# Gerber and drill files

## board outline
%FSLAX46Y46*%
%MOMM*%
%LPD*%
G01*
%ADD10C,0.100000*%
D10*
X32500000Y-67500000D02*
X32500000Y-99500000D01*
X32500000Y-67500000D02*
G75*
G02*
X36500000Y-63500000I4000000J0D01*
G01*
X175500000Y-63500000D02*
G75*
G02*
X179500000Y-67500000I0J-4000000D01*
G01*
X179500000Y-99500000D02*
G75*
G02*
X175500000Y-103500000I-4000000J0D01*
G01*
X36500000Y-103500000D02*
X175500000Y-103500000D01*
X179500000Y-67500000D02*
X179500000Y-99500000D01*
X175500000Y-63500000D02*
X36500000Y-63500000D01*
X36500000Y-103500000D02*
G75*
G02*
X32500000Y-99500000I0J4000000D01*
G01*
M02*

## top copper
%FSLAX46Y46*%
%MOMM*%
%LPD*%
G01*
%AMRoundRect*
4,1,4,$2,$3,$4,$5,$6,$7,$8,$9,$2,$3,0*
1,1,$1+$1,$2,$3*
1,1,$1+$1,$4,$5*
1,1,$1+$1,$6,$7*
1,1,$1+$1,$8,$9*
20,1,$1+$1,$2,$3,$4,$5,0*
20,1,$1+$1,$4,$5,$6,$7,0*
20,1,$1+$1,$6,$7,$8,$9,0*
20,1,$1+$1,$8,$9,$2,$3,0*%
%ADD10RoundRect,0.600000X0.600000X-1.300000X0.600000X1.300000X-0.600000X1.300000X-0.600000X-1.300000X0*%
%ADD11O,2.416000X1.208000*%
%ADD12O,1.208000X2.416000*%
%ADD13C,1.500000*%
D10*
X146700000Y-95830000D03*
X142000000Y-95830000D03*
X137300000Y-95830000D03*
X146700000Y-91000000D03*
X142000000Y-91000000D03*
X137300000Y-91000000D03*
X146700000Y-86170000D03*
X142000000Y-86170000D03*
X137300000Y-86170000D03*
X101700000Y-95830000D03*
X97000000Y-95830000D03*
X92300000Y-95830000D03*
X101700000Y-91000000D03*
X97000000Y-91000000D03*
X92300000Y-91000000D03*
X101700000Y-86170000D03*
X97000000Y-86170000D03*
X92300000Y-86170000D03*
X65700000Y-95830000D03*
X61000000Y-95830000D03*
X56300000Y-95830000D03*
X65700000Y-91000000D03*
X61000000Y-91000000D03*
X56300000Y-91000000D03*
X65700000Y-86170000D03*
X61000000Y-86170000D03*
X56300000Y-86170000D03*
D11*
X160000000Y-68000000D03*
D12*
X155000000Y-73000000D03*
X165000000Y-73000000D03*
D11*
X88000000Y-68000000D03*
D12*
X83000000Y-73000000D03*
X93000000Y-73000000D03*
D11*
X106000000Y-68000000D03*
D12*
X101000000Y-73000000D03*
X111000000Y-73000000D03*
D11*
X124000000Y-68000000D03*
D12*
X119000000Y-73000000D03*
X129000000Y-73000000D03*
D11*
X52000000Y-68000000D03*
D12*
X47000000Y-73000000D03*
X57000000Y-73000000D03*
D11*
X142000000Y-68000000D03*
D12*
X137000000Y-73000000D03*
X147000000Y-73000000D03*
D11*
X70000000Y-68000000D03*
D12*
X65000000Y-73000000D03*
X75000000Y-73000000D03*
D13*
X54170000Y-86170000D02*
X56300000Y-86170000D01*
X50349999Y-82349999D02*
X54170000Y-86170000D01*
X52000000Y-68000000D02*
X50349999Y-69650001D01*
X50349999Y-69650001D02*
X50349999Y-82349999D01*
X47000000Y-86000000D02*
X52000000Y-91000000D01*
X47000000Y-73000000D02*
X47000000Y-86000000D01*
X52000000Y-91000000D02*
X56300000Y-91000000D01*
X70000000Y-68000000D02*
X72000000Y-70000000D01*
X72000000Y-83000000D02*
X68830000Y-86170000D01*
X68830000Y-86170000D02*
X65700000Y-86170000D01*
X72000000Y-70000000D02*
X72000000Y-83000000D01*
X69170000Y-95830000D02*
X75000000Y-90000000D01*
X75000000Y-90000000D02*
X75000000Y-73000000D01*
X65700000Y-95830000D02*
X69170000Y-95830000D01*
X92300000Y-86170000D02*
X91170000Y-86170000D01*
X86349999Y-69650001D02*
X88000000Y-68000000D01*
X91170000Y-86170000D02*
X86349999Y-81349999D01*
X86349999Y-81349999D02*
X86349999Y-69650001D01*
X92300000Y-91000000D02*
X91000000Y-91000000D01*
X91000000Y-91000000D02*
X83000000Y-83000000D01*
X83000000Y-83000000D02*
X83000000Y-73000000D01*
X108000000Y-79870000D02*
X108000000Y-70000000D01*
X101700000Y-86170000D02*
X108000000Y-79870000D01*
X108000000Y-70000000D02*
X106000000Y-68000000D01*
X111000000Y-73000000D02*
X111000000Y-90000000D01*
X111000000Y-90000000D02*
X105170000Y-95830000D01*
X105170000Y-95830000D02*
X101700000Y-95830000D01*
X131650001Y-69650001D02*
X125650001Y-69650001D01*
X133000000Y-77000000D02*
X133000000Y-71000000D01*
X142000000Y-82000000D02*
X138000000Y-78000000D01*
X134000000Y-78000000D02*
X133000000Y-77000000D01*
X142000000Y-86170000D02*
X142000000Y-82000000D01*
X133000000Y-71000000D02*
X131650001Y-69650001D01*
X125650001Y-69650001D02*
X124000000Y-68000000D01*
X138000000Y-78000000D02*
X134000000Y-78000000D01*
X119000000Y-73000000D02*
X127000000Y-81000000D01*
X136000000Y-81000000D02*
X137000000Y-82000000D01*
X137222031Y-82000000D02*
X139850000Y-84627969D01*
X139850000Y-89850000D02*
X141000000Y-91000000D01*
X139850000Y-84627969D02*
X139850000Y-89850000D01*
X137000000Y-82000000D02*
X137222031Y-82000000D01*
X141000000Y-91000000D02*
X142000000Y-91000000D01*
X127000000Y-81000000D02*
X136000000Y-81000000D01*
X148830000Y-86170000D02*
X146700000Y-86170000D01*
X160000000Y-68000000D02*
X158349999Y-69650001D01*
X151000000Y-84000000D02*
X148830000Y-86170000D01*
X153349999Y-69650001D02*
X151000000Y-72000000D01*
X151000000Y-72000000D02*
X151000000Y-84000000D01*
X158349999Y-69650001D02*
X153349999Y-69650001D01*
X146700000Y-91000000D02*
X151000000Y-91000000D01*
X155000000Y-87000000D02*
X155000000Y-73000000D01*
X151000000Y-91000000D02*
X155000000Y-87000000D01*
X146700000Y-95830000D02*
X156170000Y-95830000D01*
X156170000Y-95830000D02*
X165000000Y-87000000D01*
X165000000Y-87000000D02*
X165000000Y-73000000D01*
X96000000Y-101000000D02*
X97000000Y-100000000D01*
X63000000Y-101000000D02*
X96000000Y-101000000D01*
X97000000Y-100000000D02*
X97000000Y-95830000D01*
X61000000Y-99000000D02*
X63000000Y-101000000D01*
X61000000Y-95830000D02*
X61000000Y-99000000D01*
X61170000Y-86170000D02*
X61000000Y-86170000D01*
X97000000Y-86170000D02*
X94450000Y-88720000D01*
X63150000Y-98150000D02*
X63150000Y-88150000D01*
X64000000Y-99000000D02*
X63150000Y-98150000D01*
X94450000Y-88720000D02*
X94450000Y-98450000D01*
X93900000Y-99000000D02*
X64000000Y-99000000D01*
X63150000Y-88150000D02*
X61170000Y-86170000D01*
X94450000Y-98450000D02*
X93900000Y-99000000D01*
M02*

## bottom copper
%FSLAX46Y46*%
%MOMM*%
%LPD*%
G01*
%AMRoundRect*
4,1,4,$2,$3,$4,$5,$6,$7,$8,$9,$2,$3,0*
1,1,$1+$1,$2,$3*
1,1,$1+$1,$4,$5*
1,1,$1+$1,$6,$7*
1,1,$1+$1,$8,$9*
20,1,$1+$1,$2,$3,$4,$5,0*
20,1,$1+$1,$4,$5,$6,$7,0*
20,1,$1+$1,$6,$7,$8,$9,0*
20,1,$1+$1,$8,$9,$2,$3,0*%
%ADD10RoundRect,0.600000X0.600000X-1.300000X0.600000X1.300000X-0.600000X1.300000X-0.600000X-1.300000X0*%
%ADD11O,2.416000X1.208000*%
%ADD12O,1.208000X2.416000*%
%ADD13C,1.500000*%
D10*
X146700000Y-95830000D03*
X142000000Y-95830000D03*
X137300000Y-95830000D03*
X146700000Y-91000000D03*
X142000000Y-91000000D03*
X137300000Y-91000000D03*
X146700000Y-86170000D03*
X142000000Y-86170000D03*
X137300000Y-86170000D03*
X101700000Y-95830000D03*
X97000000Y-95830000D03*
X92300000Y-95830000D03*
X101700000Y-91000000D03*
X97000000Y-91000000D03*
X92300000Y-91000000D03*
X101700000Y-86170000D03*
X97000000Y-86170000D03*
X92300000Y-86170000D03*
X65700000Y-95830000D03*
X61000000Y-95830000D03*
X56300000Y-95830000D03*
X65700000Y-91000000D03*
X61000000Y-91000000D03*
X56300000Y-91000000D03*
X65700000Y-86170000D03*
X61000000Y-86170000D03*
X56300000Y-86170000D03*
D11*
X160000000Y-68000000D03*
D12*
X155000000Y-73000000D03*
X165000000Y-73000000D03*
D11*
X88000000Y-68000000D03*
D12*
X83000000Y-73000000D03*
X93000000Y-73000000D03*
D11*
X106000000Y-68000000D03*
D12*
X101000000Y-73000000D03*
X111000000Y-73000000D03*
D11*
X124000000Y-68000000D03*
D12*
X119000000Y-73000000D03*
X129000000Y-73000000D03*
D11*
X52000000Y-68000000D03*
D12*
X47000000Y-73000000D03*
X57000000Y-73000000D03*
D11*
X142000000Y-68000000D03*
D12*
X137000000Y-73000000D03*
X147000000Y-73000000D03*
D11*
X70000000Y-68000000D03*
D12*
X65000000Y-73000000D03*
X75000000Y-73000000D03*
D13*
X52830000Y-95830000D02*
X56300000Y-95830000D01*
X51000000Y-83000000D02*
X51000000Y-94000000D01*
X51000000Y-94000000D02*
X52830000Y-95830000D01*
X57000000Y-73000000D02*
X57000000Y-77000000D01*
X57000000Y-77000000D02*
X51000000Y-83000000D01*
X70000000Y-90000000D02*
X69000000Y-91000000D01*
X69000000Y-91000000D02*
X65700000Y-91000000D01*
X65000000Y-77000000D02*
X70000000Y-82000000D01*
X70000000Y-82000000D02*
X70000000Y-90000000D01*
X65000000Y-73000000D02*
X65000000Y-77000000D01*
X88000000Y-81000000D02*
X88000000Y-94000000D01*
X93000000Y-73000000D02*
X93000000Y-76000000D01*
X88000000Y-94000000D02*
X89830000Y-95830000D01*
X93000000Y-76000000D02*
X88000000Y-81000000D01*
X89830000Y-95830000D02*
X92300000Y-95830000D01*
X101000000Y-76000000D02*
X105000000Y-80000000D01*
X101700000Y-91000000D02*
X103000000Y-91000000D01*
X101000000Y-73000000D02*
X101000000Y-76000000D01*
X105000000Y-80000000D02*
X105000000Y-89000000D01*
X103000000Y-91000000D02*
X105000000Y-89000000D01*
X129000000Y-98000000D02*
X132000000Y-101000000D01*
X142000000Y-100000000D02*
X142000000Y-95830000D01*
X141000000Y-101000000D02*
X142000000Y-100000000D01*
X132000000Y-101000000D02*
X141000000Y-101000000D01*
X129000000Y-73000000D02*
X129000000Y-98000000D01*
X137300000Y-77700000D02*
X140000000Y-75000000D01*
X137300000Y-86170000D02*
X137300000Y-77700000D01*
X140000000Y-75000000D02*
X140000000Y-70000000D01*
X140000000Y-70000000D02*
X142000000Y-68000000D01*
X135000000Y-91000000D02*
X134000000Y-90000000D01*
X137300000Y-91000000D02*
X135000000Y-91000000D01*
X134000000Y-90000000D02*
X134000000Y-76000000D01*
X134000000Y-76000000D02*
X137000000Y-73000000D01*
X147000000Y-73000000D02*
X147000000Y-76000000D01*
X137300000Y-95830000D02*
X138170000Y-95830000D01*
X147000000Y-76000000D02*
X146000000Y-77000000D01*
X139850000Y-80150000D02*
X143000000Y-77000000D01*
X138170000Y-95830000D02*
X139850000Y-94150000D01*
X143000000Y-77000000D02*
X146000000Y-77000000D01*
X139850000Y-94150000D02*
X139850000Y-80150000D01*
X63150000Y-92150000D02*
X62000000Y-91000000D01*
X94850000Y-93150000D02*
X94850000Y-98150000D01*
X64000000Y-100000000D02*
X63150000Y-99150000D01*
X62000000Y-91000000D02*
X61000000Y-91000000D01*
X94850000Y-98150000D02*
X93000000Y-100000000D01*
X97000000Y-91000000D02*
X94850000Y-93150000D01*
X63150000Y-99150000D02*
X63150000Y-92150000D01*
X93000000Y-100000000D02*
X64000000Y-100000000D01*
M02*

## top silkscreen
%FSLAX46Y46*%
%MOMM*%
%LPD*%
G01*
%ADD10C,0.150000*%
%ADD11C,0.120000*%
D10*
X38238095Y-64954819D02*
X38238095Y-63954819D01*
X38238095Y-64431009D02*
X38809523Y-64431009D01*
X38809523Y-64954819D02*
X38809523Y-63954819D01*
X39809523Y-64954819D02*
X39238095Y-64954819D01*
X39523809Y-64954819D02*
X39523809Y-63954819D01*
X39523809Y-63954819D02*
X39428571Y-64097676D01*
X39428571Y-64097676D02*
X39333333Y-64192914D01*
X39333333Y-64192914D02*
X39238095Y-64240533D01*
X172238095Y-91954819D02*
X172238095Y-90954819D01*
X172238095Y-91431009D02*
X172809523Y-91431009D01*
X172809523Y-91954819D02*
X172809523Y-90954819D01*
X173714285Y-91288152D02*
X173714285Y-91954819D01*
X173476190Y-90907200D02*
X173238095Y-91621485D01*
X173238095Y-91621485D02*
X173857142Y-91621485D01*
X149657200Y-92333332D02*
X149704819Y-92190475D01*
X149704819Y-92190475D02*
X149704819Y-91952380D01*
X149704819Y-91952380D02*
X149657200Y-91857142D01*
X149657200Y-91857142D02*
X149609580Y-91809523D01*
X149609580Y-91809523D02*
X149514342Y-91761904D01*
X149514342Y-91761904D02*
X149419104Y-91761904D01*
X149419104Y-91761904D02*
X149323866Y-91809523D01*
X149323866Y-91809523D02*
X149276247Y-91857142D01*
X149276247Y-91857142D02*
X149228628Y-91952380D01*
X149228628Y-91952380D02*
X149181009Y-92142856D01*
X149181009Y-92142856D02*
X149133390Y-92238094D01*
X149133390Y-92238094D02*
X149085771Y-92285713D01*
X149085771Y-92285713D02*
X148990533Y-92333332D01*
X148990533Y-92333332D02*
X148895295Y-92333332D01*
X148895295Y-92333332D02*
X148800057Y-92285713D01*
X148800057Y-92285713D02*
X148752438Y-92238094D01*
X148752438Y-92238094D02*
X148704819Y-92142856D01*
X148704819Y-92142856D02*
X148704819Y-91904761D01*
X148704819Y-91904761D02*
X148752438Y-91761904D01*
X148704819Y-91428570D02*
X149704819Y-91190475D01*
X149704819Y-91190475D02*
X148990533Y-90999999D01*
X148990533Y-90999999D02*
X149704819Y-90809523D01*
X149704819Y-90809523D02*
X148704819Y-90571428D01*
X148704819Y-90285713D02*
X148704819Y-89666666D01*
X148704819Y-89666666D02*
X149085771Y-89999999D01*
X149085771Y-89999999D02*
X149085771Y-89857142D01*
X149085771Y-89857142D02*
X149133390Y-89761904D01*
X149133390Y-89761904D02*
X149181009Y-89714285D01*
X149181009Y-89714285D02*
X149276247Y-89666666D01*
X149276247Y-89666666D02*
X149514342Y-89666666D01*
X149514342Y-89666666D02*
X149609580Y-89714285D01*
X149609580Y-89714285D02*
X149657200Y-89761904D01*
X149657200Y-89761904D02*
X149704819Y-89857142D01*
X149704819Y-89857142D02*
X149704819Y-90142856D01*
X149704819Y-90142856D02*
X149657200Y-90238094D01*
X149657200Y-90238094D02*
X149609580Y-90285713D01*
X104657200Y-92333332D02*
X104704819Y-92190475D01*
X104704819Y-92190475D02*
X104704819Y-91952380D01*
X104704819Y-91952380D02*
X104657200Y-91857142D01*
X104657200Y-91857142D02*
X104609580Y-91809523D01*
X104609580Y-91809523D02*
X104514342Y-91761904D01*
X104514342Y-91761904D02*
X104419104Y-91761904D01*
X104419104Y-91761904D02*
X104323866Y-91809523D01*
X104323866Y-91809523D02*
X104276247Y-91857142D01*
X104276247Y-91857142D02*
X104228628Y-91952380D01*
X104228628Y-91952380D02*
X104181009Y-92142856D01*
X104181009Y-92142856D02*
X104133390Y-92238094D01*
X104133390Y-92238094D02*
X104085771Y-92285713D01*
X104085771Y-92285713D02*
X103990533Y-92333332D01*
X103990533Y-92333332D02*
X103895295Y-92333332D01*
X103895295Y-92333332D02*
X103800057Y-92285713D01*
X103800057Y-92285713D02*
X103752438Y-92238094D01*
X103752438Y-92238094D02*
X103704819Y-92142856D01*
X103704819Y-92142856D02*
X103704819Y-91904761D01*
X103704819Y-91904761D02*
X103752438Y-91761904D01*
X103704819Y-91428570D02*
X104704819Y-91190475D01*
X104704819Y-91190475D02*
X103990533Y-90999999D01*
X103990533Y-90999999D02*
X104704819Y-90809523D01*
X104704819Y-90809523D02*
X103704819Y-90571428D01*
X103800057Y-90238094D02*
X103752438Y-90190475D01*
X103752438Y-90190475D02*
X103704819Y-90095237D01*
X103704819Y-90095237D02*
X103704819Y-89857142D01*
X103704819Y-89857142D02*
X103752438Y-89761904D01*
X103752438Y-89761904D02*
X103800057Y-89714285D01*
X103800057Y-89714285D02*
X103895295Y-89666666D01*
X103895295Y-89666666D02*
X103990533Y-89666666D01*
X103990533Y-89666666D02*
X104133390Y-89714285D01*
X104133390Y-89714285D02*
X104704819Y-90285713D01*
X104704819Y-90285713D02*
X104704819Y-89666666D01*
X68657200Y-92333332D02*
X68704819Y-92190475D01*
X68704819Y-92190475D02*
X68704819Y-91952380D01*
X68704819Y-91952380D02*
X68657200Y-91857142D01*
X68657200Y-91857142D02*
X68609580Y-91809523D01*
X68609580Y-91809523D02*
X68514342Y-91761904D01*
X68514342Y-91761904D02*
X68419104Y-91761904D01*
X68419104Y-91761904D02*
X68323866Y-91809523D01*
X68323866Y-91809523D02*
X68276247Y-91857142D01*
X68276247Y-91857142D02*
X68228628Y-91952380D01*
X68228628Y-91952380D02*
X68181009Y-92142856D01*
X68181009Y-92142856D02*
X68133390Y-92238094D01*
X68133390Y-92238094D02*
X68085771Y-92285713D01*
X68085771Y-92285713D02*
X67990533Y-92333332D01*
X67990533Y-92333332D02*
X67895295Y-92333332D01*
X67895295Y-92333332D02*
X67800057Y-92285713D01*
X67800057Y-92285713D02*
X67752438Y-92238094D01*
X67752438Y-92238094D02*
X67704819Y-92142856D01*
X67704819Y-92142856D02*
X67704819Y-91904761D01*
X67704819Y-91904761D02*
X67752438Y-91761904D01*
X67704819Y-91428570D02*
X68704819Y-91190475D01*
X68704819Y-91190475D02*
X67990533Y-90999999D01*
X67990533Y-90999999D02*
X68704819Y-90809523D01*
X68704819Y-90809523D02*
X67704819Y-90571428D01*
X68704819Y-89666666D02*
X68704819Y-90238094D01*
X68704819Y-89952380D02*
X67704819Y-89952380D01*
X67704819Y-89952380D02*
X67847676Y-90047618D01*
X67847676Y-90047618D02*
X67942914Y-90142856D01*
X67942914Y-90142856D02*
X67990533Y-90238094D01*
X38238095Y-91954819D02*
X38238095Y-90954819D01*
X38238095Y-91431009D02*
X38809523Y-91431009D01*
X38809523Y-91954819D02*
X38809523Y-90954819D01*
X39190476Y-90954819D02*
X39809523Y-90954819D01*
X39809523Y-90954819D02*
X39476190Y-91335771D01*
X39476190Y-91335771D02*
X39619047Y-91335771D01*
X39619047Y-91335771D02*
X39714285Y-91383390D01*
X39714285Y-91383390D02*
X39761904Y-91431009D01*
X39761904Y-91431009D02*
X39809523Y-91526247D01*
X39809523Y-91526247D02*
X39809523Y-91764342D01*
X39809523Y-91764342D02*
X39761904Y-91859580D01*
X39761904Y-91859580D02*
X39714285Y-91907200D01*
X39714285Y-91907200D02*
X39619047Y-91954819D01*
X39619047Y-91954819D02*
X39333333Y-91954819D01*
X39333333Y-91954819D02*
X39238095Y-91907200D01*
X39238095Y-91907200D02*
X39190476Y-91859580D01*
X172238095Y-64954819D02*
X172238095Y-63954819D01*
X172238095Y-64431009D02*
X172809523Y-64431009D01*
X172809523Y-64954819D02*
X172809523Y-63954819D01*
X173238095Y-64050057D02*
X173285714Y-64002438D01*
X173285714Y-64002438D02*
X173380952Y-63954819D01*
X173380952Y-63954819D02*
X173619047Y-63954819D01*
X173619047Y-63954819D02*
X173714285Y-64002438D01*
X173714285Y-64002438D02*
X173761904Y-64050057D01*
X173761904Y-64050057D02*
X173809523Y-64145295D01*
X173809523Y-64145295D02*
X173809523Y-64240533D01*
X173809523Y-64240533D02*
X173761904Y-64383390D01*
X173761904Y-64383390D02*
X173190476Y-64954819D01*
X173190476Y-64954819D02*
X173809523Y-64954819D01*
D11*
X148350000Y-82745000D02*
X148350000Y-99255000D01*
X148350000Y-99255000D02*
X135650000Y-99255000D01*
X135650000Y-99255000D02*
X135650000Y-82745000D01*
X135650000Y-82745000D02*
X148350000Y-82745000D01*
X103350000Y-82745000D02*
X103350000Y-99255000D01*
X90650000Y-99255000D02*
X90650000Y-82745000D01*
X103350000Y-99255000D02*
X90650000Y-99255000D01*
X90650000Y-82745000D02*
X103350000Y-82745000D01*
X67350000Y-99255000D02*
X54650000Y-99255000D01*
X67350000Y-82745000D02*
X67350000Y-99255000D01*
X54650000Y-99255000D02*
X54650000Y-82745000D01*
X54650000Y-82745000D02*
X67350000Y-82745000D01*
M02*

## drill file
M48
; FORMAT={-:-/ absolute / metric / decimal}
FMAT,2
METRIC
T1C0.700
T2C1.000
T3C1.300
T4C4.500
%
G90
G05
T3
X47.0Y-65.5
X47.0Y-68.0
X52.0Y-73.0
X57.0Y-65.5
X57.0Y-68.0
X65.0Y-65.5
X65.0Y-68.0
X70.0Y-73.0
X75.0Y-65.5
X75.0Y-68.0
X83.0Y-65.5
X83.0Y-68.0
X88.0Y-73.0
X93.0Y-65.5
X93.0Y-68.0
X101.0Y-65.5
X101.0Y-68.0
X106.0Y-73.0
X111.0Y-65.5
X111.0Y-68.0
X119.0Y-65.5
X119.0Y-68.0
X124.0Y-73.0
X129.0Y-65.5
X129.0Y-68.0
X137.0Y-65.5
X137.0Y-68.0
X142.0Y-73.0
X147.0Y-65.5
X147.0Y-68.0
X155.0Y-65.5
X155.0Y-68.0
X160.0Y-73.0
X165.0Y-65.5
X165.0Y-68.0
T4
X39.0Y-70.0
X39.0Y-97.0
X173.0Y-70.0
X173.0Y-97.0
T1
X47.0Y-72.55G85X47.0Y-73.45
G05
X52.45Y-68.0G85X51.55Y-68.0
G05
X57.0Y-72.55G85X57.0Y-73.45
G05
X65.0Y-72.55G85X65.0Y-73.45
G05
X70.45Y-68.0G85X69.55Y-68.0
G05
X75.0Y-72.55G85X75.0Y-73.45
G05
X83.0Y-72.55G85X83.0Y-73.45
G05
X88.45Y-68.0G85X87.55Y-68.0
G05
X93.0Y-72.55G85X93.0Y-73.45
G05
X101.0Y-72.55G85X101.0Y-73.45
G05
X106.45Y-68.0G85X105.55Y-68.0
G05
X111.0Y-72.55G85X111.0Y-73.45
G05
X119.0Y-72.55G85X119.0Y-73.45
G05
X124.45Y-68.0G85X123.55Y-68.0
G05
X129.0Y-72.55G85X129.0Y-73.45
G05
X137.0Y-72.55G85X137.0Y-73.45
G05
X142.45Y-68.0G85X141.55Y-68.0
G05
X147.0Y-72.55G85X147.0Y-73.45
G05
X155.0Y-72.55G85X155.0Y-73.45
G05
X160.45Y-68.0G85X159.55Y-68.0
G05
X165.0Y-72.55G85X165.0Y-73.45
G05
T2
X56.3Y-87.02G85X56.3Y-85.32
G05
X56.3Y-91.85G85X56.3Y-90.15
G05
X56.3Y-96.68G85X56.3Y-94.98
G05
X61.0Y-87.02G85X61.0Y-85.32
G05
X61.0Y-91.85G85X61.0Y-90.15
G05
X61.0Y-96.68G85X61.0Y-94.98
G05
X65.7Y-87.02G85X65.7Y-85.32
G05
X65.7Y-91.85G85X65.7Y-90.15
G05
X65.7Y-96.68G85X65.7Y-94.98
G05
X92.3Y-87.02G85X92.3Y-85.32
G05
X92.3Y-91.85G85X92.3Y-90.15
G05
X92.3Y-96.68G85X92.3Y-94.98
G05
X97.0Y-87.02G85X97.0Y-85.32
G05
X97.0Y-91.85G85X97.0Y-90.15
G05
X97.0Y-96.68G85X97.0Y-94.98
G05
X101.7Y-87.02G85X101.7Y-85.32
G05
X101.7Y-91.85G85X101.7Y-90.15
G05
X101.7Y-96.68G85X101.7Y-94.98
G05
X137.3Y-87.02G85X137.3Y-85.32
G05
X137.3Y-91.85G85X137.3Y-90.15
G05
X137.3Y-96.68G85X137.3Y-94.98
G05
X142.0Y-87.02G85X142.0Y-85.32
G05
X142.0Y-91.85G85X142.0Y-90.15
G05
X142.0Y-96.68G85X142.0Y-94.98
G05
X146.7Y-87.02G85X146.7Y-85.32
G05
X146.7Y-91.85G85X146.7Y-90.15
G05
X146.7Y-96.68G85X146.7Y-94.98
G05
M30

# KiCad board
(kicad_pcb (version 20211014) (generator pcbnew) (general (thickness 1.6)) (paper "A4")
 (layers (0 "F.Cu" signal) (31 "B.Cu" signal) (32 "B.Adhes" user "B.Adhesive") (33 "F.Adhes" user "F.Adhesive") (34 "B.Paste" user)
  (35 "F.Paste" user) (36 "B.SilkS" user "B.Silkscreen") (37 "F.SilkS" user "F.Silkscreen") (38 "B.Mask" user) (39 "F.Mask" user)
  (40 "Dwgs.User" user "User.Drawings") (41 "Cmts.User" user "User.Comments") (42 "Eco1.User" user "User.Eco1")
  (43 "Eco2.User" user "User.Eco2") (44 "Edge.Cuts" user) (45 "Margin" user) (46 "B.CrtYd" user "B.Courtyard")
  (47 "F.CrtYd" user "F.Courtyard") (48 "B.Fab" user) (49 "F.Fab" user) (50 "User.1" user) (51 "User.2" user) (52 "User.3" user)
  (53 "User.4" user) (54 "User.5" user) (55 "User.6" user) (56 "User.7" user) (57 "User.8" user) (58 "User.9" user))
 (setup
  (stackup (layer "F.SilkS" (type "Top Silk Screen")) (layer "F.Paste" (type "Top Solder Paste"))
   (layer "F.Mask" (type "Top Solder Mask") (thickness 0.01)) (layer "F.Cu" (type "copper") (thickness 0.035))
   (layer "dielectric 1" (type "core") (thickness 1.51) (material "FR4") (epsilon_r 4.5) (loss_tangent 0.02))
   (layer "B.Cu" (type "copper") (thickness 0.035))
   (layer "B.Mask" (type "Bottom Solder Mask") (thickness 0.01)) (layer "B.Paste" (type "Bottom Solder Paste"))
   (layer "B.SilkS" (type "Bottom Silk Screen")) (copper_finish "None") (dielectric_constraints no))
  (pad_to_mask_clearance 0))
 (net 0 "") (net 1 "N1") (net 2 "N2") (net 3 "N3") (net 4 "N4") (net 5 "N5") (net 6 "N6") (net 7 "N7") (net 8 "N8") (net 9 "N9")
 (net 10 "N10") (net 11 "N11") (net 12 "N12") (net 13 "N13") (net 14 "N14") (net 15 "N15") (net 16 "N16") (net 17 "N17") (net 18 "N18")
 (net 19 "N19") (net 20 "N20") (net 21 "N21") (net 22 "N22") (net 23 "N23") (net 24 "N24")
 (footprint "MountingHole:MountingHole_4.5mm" (layer "F.Cu") (at 39 70)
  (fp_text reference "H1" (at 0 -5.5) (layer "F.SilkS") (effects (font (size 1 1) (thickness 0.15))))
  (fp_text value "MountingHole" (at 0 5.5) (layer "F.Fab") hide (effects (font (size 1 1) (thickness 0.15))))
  (pad "" np_thru_hole circle (at 0 0) (size 4.5 4.5) (drill 4.5) (layers *.Cu *.Mask)))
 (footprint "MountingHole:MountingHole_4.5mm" (layer "F.Cu") (at 173 97)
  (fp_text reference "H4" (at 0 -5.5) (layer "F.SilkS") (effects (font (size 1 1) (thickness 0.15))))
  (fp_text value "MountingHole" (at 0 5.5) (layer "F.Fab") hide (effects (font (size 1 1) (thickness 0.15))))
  (pad "" np_thru_hole circle (at 0 0) (size 4.5 4.5) (drill 4.5) (layers *.Cu *.Mask)))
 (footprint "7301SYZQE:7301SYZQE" (layer "F.Cu") (at 142 91 90)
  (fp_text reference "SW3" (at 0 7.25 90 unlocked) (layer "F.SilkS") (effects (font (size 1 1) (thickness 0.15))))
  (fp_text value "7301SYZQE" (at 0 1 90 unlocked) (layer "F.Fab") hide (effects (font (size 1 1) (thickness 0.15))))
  (fp_line (start 8.255 6.35) (end -8.255 6.35) (layer "F.SilkS") (width 0.12))
  (fp_line (start -8.255 6.35) (end -8.255 -6.35) (layer "F.SilkS") (width 0.12))
  (fp_line (start -8.255 -6.35) (end 8.255 -6.35) (layer "F.SilkS") (width 0.12))
  (fp_line (start 8.255 -6.35) (end 8.255 6.35) (layer "F.SilkS") (width 0.12))
  (pad "1" thru_hole roundrect (at -4.83 4.7 90) (size 3.8 2.4) (drill oval 2.7 1) (layers *.Cu *.Mask) (roundrect_rratio 0.25) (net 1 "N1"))
  (pad "2" thru_hole roundrect (at -4.83 0 90) (size 3.8 2.4) (drill oval 2.7 1) (layers *.Cu *.Mask) (roundrect_rratio 0.25) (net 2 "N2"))
  (pad "3" thru_hole roundrect (at -4.83 -4.7 90) (size 3.8 2.4) (drill oval 2.7 1) (layers *.Cu *.Mask) (roundrect_rratio 0.25)
   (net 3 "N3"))
  (pad "4" thru_hole roundrect (at 0 4.7 90) (size 3.8 2.4) (drill oval 2.7 1) (layers *.Cu *.Mask) (roundrect_rratio 0.25) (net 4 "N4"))
  (pad "5" thru_hole roundrect (at 0 0 90) (size 3.8 2.4) (drill oval 2.7 1) (layers *.Cu *.Mask) (roundrect_rratio 0.25) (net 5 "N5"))
  (pad "6" thru_hole roundrect (at 0 -4.7 90) (size 3.8 2.4) (drill oval 2.7 1) (layers *.Cu *.Mask) (roundrect_rratio 0.25) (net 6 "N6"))
  (pad "7" thru_hole roundrect (at 4.83 4.7 90) (size 3.8 2.4) (drill oval 2.7 1) (layers *.Cu *.Mask) (roundrect_rratio 0.25) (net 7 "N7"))
  (pad "8" thru_hole roundrect (at 4.83 0 90) (size 3.8 2.4) (drill oval 2.7 1) (layers *.Cu *.Mask) (roundrect_rratio 0.25) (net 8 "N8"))
  (pad "9" thru_hole roundrect (at 4.83 -4.7 90) (size 3.8 2.4) (drill oval 2.7 1) (layers *.Cu *.Mask) (roundrect_rratio 0.25) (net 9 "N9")))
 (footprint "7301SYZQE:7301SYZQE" (layer "F.Cu") (at 97 91 90)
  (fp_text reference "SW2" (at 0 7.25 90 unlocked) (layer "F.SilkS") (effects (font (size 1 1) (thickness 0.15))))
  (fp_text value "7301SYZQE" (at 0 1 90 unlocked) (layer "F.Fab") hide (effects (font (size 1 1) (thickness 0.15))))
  (fp_line (start 8.255 6.35) (end -8.255 6.35) (layer "F.SilkS") (width 0.12))
  (fp_line (start -8.255 -6.35) (end 8.255 -6.35) (layer "F.SilkS") (width 0.12))
  (fp_line (start -8.255 6.35) (end -8.255 -6.35) (layer "F.SilkS") (width 0.12))
  (fp_line (start 8.255 -6.35) (end 8.255 6.35) (layer "F.SilkS") (width 0.12))
  (pad "1" thru_hole roundrect (at -4.83 4.7 90) (size 3.8 2.4) (drill oval 2.7 1) (layers *.Cu *.Mask) (roundrect_rratio 0.25)
   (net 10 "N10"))
  (pad "2" thru_hole roundrect (at -4.83 0 90) (size 3.8 2.4) (drill oval 2.7 1) (layers *.Cu *.Mask) (roundrect_rratio 0.25) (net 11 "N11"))
  (pad "3" thru_hole roundrect (at -4.83 -4.7 90) (size 3.8 2.4) (drill oval 2.7 1) (layers *.Cu *.Mask) (roundrect_rratio 0.25)
   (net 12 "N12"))
  (pad "4" thru_hole roundrect (at 0 4.7 90) (size 3.8 2.4) (drill oval 2.7 1) (layers *.Cu *.Mask) (roundrect_rratio 0.25) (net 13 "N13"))
  (pad "5" thru_hole roundrect (at 0 0 90) (size 3.8 2.4) (drill oval 2.7 1) (layers *.Cu *.Mask) (roundrect_rratio 0.25) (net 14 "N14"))
  (pad "6" thru_hole roundrect (at 0 -4.7 90) (size 3.8 2.4) (drill oval 2.7 1) (layers *.Cu *.Mask) (roundrect_rratio 0.25) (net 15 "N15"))
  (pad "7" thru_hole roundrect (at 4.83 4.7 90) (size 3.8 2.4) (drill oval 2.7 1) (layers *.Cu *.Mask) (roundrect_rratio 0.25)
   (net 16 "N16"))
  (pad "8" thru_hole roundrect (at 4.83 0 90) (size 3.8 2.4) (drill oval 2.7 1) (layers *.Cu *.Mask) (roundrect_rratio 0.25) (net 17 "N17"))
  (pad "9" thru_hole roundrect (at 4.83 -4.7 90) (size 3.8 2.4) (drill oval 2.7 1) (layers *.Cu *.Mask) (roundrect_rratio 0.25)
   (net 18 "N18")))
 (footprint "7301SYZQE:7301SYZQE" (layer "F.Cu") (at 61 91 90)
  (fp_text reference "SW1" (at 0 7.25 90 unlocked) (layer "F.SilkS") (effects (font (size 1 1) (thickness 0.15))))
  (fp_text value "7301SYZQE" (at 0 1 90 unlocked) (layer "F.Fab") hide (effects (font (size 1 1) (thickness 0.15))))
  (fp_line (start -8.255 6.35) (end -8.255 -6.35) (layer "F.SilkS") (width 0.12))
  (fp_line (start 8.255 6.35) (end -8.255 6.35) (layer "F.SilkS") (width 0.12))
  (fp_line (start -8.255 -6.35) (end 8.255 -6.35) (layer "F.SilkS") (width 0.12))
  (fp_line (start 8.255 -6.35) (end 8.255 6.35) (layer "F.SilkS") (width 0.12))
  (pad "1" thru_hole roundrect (at -4.83 4.7 90) (size 3.8 2.4) (drill oval 2.7 1) (layers *.Cu *.Mask) (roundrect_rratio 0.25)
   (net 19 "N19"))
  (pad "2" thru_hole roundrect (at -4.83 0 90) (size 3.8 2.4) (drill oval 2.7 1) (layers *.Cu *.Mask) (roundrect_rratio 0.25) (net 11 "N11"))
  (pad "3" thru_hole roundrect (at -4.83 -4.7 90) (size 3.8 2.4) (drill oval 2.7 1) (layers *.Cu *.Mask) (roundrect_rratio 0.25)
   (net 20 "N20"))
  (pad "4" thru_hole roundrect (at 0 4.7 90) (size 3.8 2.4) (drill oval 2.7 1) (layers *.Cu *.Mask) (roundrect_rratio 0.25) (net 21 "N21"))
  (pad "5" thru_hole roundrect (at 0 0 90) (size 3.8 2.4) (drill oval 2.7 1) (layers *.Cu *.Mask) (roundrect_rratio 0.25) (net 14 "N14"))
  (pad "6" thru_hole roundrect (at 0 -4.7 90) (size 3.8 2.4) (drill oval 2.7 1) (layers *.Cu *.Mask) (roundrect_rratio 0.25) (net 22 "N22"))
  (pad "7" thru_hole roundrect (at 4.83 4.7 90) (size 3.8 2.4) (drill oval 2.7 1) (layers *.Cu *.Mask) (roundrect_rratio 0.25)
   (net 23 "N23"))
  (pad "8" thru_hole roundrect (at 4.83 0 90) (size 3.8 2.4) (drill oval 2.7 1) (layers *.Cu *.Mask) (roundrect_rratio 0.25) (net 17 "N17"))
  (pad "9" thru_hole roundrect (at 4.83 -4.7 90) (size 3.8 2.4) (drill oval 2.7 1) (layers *.Cu *.Mask) (roundrect_rratio 0.25)
   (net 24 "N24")))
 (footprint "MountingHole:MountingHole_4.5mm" (layer "F.Cu") (at 39 97)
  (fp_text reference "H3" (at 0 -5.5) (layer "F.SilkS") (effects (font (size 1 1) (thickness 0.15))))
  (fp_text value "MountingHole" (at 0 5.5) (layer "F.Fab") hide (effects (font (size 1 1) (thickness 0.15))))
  (pad "" np_thru_hole circle (at 0 0) (size 4.5 4.5) (drill 4.5) (layers *.Cu *.Mask)))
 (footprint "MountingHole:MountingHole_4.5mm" (layer "F.Cu") (at 173 70)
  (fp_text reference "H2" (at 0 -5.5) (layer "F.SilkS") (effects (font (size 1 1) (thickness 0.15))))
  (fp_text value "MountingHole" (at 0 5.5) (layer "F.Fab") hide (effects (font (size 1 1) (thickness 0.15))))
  (pad "" np_thru_hole circle (at 0 0) (size 4.5 4.5) (drill 4.5) (layers *.Cu *.Mask)))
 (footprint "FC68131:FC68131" (layer "B.Cu") (at 160 68 -90)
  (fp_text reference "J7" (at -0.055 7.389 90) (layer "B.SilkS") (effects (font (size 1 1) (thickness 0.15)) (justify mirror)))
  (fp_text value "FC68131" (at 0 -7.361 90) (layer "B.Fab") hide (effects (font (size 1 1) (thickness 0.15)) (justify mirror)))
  (pad "" np_thru_hole circle (at 0 5 270) (size 1.3 1.3) (drill 1.3) (layers *.Cu *.Mask))
  (pad "" np_thru_hole circle (at 5 0 270) (size 1.3 1.3) (drill 1.3) (layers *.Cu *.Mask))
  (pad "" np_thru_hole circle (at 0 -5 270) (size 1.3 1.3) (drill 1.3) (layers *.Cu *.Mask))
  (pad "" np_thru_hole circle (at -2.5 -5 270) (size 1.3 1.3) (drill 1.3) (layers *.Cu *.Mask))
  (pad "" np_thru_hole circle (at -2.5 5 270) (size 1.3 1.3) (drill 1.3) (layers *.Cu *.Mask))
  (pad "1" thru_hole oval (at 0 0 270) (size 1.208 2.416) (drill oval 0.7 1.6) (layers *.Cu *.Mask) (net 7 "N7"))
  (pad "2" thru_hole oval (at 5 5 270) (size 2.416 1.208) (drill oval 1.6 0.7) (layers *.Cu *.Mask) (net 4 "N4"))
  (pad "5" thru_hole oval (at 5 -5 270) (size 2.416 1.208) (drill oval 1.6 0.7) (layers *.Cu *.Mask) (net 1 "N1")))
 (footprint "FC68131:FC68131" (layer "B.Cu") (at 88 68 -90)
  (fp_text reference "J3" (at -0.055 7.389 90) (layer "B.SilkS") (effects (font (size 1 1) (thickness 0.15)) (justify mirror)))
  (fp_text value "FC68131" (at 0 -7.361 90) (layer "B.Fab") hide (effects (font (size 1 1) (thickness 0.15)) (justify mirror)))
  (pad "" np_thru_hole circle (at -2.5 -5 270) (size 1.3 1.3) (drill 1.3) (layers *.Cu *.Mask))
  (pad "" np_thru_hole circle (at 5 0 270) (size 1.3 1.3) (drill 1.3) (layers *.Cu *.Mask))
  (pad "" np_thru_hole circle (at -2.5 5 270) (size 1.3 1.3) (drill 1.3) (layers *.Cu *.Mask))
  (pad "" np_thru_hole circle (at 0 -5 270) (size 1.3 1.3) (drill 1.3) (layers *.Cu *.Mask))
  (pad "" np_thru_hole circle (at 0 5 270) (size 1.3 1.3) (drill 1.3) (layers *.Cu *.Mask))
  (pad "1" thru_hole oval (at 0 0 270) (size 1.208 2.416) (drill oval 0.7 1.6) (layers *.Cu *.Mask) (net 18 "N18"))
  (pad "2" thru_hole oval (at 5 5 270) (size 2.416 1.208) (drill oval 1.6 0.7) (layers *.Cu *.Mask) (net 15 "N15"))
  (pad "5" thru_hole oval (at 5 -5 270) (size 2.416 1.208) (drill oval 1.6 0.7) (layers *.Cu *.Mask) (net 12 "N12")))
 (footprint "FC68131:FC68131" (layer "B.Cu") (at 106 68 -90)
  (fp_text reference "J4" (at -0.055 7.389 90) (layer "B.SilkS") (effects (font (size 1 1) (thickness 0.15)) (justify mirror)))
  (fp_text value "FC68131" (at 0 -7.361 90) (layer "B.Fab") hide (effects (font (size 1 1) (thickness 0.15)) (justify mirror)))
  (pad "" np_thru_hole circle (at 0 -5 270) (size 1.3 1.3) (drill 1.3) (layers *.Cu *.Mask))
  (pad "" np_thru_hole circle (at -2.5 5 270) (size 1.3 1.3) (drill 1.3) (layers *.Cu *.Mask))
  (pad "" np_thru_hole circle (at 0 5 270) (size 1.3 1.3) (drill 1.3) (layers *.Cu *.Mask))
  (pad "" np_thru_hole circle (at 5 0 270) (size 1.3 1.3) (drill 1.3) (layers *.Cu *.Mask))
  (pad "" np_thru_hole circle (at -2.5 -5 270) (size 1.3 1.3) (drill 1.3) (layers *.Cu *.Mask))
  (pad "1" thru_hole oval (at 0 0 270) (size 1.208 2.416) (drill oval 0.7 1.6) (layers *.Cu *.Mask) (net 16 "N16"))
  (pad "2" thru_hole oval (at 5 5 270) (size 2.416 1.208) (drill oval 1.6 0.7) (layers *.Cu *.Mask) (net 13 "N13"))
  (pad "5" thru_hole oval (at 5 -5 270) (size 2.416 1.208) (drill oval 1.6 0.7) (layers *.Cu *.Mask) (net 10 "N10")))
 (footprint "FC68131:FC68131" (layer "B.Cu") (at 124 68 -90)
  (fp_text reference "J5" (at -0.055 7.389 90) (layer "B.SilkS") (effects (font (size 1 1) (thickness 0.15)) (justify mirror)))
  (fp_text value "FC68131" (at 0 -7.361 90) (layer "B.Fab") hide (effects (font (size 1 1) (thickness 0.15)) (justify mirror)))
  (pad "" np_thru_hole circle (at 5 0 270) (size 1.3 1.3) (drill 1.3) (layers *.Cu *.Mask))
  (pad "" np_thru_hole circle (at 0 -5 270) (size 1.3 1.3) (drill 1.3) (layers *.Cu *.Mask))
  (pad "" np_thru_hole circle (at 0 5 270) (size 1.3 1.3) (drill 1.3) (layers *.Cu *.Mask))
  (pad "" np_thru_hole circle (at -2.5 -5 270) (size 1.3 1.3) (drill 1.3) (layers *.Cu *.Mask))
  (pad "" np_thru_hole circle (at -2.5 5 270) (size 1.3 1.3) (drill 1.3) (layers *.Cu *.Mask))
  (pad "1" thru_hole oval (at 0 0 270) (size 1.208 2.416) (drill oval 0.7 1.6) (layers *.Cu *.Mask) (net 8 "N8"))
  (pad "2" thru_hole oval (at 5 5 270) (size 2.416 1.208) (drill oval 1.6 0.7) (layers *.Cu *.Mask) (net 5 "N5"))
  (pad "5" thru_hole oval (at 5 -5 270) (size 2.416 1.208) (drill oval 1.6 0.7) (layers *.Cu *.Mask) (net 2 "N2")))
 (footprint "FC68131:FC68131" (layer "B.Cu") (at 52 68 -90)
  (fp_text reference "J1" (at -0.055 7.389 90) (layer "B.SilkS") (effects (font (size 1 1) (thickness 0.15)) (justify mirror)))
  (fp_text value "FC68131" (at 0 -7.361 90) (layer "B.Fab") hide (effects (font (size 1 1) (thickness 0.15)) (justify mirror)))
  (pad "" np_thru_hole circle (at 0 5 270) (size 1.3 1.3) (drill 1.3) (layers *.Cu *.Mask))
  (pad "" np_thru_hole circle (at -2.5 -5 270) (size 1.3 1.3) (drill 1.3) (layers *.Cu *.Mask))
  (pad "" np_thru_hole circle (at -2.5 5 270) (size 1.3 1.3) (drill 1.3) (layers *.Cu *.Mask))
  (pad "" np_thru_hole circle (at 0 -5 270) (size 1.3 1.3) (drill 1.3) (layers *.Cu *.Mask))
  (pad "" np_thru_hole circle (at 5 0 270) (size 1.3 1.3) (drill 1.3) (layers *.Cu *.Mask))
  (pad "1" thru_hole oval (at 0 0 270) (size 1.208 2.416) (drill oval 0.7 1.6) (layers *.Cu *.Mask) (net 24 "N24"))
  (pad "2" thru_hole oval (at 5 5 270) (size 2.416 1.208) (drill oval 1.6 0.7) (layers *.Cu *.Mask) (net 22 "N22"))
  (pad "5" thru_hole oval (at 5 -5 270) (size 2.416 1.208) (drill oval 1.6 0.7) (layers *.Cu *.Mask) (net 20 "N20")))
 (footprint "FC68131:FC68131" (layer "B.Cu") (at 142 68 -90)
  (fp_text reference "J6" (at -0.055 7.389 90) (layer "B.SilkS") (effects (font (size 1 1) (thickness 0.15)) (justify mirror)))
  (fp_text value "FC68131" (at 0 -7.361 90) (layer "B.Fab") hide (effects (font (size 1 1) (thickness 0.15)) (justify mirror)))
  (pad "" np_thru_hole circle (at 0 5 270) (size 1.3 1.3) (drill 1.3) (layers *.Cu *.Mask))
  (pad "" np_thru_hole circle (at 0 -5 270) (size 1.3 1.3) (drill 1.3) (layers *.Cu *.Mask))
  (pad "" np_thru_hole circle (at -2.5 5 270) (size 1.3 1.3) (drill 1.3) (layers *.Cu *.Mask))
  (pad "" np_thru_hole circle (at -2.5 -5 270) (size 1.3 1.3) (drill 1.3) (layers *.Cu *.Mask))
  (pad "" np_thru_hole circle (at 5 0 270) (size 1.3 1.3) (drill 1.3) (layers *.Cu *.Mask))
  (pad "1" thru_hole oval (at 0 0 270) (size 1.208 2.416) (drill oval 0.7 1.6) (layers *.Cu *.Mask) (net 9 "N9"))
  (pad "2" thru_hole oval (at 5 5 270) (size 2.416 1.208) (drill oval 1.6 0.7) (layers *.Cu *.Mask) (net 6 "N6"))
  (pad "5" thru_hole oval (at 5 -5 270) (size 2.416 1.208) (drill oval 1.6 0.7) (layers *.Cu *.Mask) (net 3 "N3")))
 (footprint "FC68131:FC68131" (layer "B.Cu") (at 70 68 -90)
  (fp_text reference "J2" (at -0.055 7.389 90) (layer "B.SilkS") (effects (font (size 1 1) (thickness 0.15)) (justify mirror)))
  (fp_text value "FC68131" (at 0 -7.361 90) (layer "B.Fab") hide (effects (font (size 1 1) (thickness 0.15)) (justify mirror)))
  (pad "" np_thru_hole circle (at -2.5 -5 270) (size 1.3 1.3) (drill 1.3) (layers *.Cu *.Mask))
  (pad "" np_thru_hole circle (at 5 0 270) (size 1.3 1.3) (drill 1.3) (layers *.Cu *.Mask))
  (pad "" np_thru_hole circle (at -2.5 5 270) (size 1.3 1.3) (drill 1.3) (layers *.Cu *.Mask))
  (pad "" np_thru_hole circle (at 0 -5 270) (size 1.3 1.3) (drill 1.3) (layers *.Cu *.Mask))
  (pad "" np_thru_hole circle (at 0 5 270) (size 1.3 1.3) (drill 1.3) (layers *.Cu *.Mask))
  (pad "1" thru_hole oval (at 0 0 270) (size 1.208 2.416) (drill oval 0.7 1.6) (layers *.Cu *.Mask) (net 23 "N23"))
  (pad "2" thru_hole oval (at 5 5 270) (size 2.416 1.208) (drill oval 1.6 0.7) (layers *.Cu *.Mask) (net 21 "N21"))
  (pad "5" thru_hole oval (at 5 -5 270) (size 2.416 1.208) (drill oval 1.6 0.7) (layers *.Cu *.Mask) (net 19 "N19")))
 (gr_line (start 32.5 67.5) (end 32.5 99.5) (layer "Edge.Cuts") (width 0.1))
 (gr_arc (start 32.5 67.5) (mid 33.671573 64.671573) (end 36.5 63.5) (layer "Edge.Cuts") (width 0.1))
 (gr_arc (start 175.5 63.5) (mid 178.328427 64.671573) (end 179.5 67.5) (layer "Edge.Cuts") (width 0.1))
 (gr_arc (start 179.5 99.5) (mid 178.328427 102.328427) (end 175.5 103.5) (layer "Edge.Cuts") (width 0.1))
 (gr_line (start 36.5 103.5) (end 175.5 103.5) (layer "Edge.Cuts") (width 0.1))
 (gr_line (start 179.5 67.5) (end 179.5 99.5) (layer "Edge.Cuts") (width 0.1))
 (gr_line (start 175.5 63.5) (end 36.5 63.5) (layer "Edge.Cuts") (width 0.1))
 (gr_arc (start 36.5 103.5) (mid 33.671573 102.328427) (end 32.5 99.5) (layer "Edge.Cuts") (width 0.1))
 (segment (start 54.17 86.17) (end 56.3 86.17) (width 1.5) (layer "F.Cu") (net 24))
 (segment (start 50.349999 82.349999) (end 54.17 86.17) (width 1.5) (layer "F.Cu") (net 24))
 (segment (start 52 68) (end 50.349999 69.650001) (width 1.5) (layer "F.Cu") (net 24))
 (segment (start 50.349999 69.650001) (end 50.349999 82.349999) (width 1.5) (layer "F.Cu") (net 24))
 (segment (start 47 86) (end 52 91) (width 1.5) (layer "F.Cu") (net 22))
 (segment (start 47 73) (end 47 86) (width 1.5) (layer "F.Cu") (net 22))
 (segment (start 52 91) (end 56.3 91) (width 1.5) (layer "F.Cu") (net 22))
 (segment (start 52.83 95.83) (end 56.3 95.83) (width 1.5) (layer "B.Cu") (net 20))
 (segment (start 51 83) (end 51 94) (width 1.5) (layer "B.Cu") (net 20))
 (segment (start 51 94) (end 52.83 95.83) (width 1.5) (layer "B.Cu") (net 20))
 (segment (start 57 73) (end 57 77) (width 1.5) (layer "B.Cu") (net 20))
 (segment (start 57 77) (end 51 83) (width 1.5) (layer "B.Cu") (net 20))
 (segment (start 70 68) (end 72 70) (width 1.5) (layer "F.Cu") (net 23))
 (segment (start 72 83) (end 68.83 86.17) (width 1.5) (layer "F.Cu") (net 23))
 (segment (start 68.83 86.17) (end 65.7 86.17) (width 1.5) (layer "F.Cu") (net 23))
 (segment (start 72 70) (end 72 83) (width 1.5) (layer "F.Cu") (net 23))
 (segment (start 70 90) (end 69 91) (width 1.5) (layer "B.Cu") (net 21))
 (segment (start 69 91) (end 65.7 91) (width 1.5) (layer "B.Cu") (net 21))
 (segment (start 65 77) (end 70 82) (width 1.5) (layer "B.Cu") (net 21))
 (segment (start 70 82) (end 70 90) (width 1.5) (layer "B.Cu") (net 21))
 (segment (start 65 73) (end 65 77) (width 1.5) (layer "B.Cu") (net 21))
 (segment (start 69.17 95.83) (end 75 90) (width 1.5) (layer "F.Cu") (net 19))
 (segment (start 75 90) (end 75 73) (width 1.5) (layer "F.Cu") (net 19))
 (segment (start 65.7 95.83) (end 69.17 95.83) (width 1.5) (layer "F.Cu") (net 19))
 (segment (start 92.3 86.17) (end 91.17 86.17) (width 1.5) (layer "F.Cu") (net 18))
 (segment (start 86.349999 69.650001) (end 88 68) (width 1.5) (layer "F.Cu") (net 18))
 (segment (start 91.17 86.17) (end 86.349999 81.349999) (width 1.5) (layer "F.Cu") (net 18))
 (segment (start 86.349999 81.349999) (end 86.349999 69.650001) (width 1.5) (layer "F.Cu") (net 18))
 (segment (start 92.3 91) (end 91 91) (width 1.5) (layer "F.Cu") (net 15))
 (segment (start 91 91) (end 83 83) (width 1.5) (layer "F.Cu") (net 15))
 (segment (start 83 83) (end 83 73) (width 1.5) (layer "F.Cu") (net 15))
 (segment (start 88 81) (end 88 94) (width 1.5) (layer "B.Cu") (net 12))
 (segment (start 93 73) (end 93 76) (width 1.5) (layer "B.Cu") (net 12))
 (segment (start 88 94) (end 89.83 95.83) (width 1.5) (layer "B.Cu") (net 12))
 (segment (start 93 76) (end 88 81) (width 1.5) (layer "B.Cu") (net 12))
 (segment (start 89.83 95.83) (end 92.3 95.83) (width 1.5) (layer "B.Cu") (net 12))
 (segment (start 108 79.87) (end 108 70) (width 1.5) (layer "F.Cu") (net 16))
 (segment (start 101.7 86.17) (end 108 79.87) (width 1.5) (layer "F.Cu") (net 16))
 (segment (start 108 70) (end 106 68) (width 1.5) (layer "F.Cu") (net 16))
 (segment (start 101 76) (end 105 80) (width 1.5) (layer "B.Cu") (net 13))
 (segment (start 101.7 91) (end 103 91) (width 1.5) (layer "B.Cu") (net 13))
 (segment (start 101 73) (end 101 76) (width 1.5) (layer "B.Cu") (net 13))
 (segment (start 105 80) (end 105 89) (width 1.5) (layer "B.Cu") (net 13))
 (segment (start 103 91) (end 105 89) (width 1.5) (layer "B.Cu") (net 13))
 (segment (start 111 73) (end 111 90) (width 1.5) (layer "F.Cu") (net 10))
 (segment (start 111 90) (end 105.17 95.83) (width 1.5) (layer "F.Cu") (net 10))
 (segment (start 105.17 95.83) (end 101.7 95.83) (width 1.5) (layer "F.Cu") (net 10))
 (segment (start 131.650001 69.650001) (end 125.650001 69.650001) (width 1.5) (layer "F.Cu") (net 8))
 (segment (start 133 77) (end 133 71) (width 1.5) (layer "F.Cu") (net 8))
 (segment (start 142 82) (end 138 78) (width 1.5) (layer "F.Cu") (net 8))
 (segment (start 134 78) (end 133 77) (width 1.5) (layer "F.Cu") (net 8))
 (segment (start 142 86.17) (end 142 82) (width 1.5) (layer "F.Cu") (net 8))
 (segment (start 133 71) (end 131.650001 69.650001) (width 1.5) (layer "F.Cu") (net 8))
 (segment (start 125.650001 69.650001) (end 124 68) (width 1.5) (layer "F.Cu") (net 8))
 (segment (start 138 78) (end 134 78) (width 1.5) (layer "F.Cu") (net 8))
 (segment (start 119 73) (end 127 81) (width 1.5) (layer "F.Cu") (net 5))
 (segment (start 136 81) (end 137 82) (width 1.5) (layer "F.Cu") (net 5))
 (segment (start 137.222031 82) (end 139.85 84.627969) (width 1.5) (layer "F.Cu") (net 5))
 (segment (start 139.85 89.85) (end 141 91) (width 1.5) (layer "F.Cu") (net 5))
 (segment (start 139.85 84.627969) (end 139.85 89.85) (width 1.5) (layer "F.Cu") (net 5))
 (segment (start 137 82) (end 137.222031 82) (width 1.5) (layer "F.Cu") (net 5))
 (segment (start 141 91) (end 142 91) (width 1.5) (layer "F.Cu") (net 5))
 (segment (start 127 81) (end 136 81) (width 1.5) (layer "F.Cu") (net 5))
 (segment (start 129 98) (end 132 101) (width 1.5) (layer "B.Cu") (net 2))
 (segment (start 142 100) (end 142 95.83) (width 1.5) (layer "B.Cu") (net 2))
 (segment (start 141 101) (end 142 100) (width 1.5) (layer "B.Cu") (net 2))
 (segment (start 132 101) (end 141 101) (width 1.5) (layer "B.Cu") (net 2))
 (segment (start 129 73) (end 129 98) (width 1.5) (layer "B.Cu") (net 2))
 (segment (start 137.3 77.7) (end 140 75) (width 1.5) (layer "B.Cu") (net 9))
 (segment (start 137.3 86.17) (end 137.3 77.7) (width 1.5) (layer "B.Cu") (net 9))
 (segment (start 140 75) (end 140 70) (width 1.5) (layer "B.Cu") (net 9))
 (segment (start 140 70) (end 142 68) (width 1.5) (layer "B.Cu") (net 9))
 (segment (start 135 91) (end 134 90) (width 1.5) (layer "B.Cu") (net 6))
 (segment (start 137.3 91) (end 135 91) (width 1.5) (layer "B.Cu") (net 6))
 (segment (start 134 90) (end 134 76) (width 1.5) (layer "B.Cu") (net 6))
 (segment (start 134 76) (end 137 73) (width 1.5) (layer "B.Cu") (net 6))
 (segment (start 147 73) (end 147 76) (width 1.5) (layer "B.Cu") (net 3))
 (segment (start 137.3 95.83) (end 138.17 95.83) (width 1.5) (layer "B.Cu") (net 3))
 (segment (start 147 76) (end 146 77) (width 1.5) (layer "B.Cu") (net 3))
 (segment (start 139.85 80.15) (end 143 77) (width 1.5) (layer "B.Cu") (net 3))
 (segment (start 138.17 95.83) (end 139.85 94.15) (width 1.5) (layer "B.Cu") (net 3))
 (segment (start 143 77) (end 146 77) (width 1.5) (layer "B.Cu") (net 3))
 (segment (start 139.85 94.15) (end 139.85 80.15) (width 1.5) (layer "B.Cu") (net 3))
 (segment (start 148.83 86.17) (end 146.7 86.17) (width 1.5) (layer "F.Cu") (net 7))
 (segment (start 160 68) (end 158.349999 69.650001) (width 1.5) (layer "F.Cu") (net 7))
 (segment (start 151 84) (end 148.83 86.17) (width 1.5) (layer "F.Cu") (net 7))
 (segment (start 153.349999 69.650001) (end 151 72) (width 1.5) (layer "F.Cu") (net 7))
 (segment (start 151 72) (end 151 84) (width 1.5) (layer "F.Cu") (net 7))
 (segment (start 158.349999 69.650001) (end 153.349999 69.650001) (width 1.5) (layer "F.Cu") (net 7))
 (segment (start 146.7 91) (end 151 91) (width 1.5) (layer "F.Cu") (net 4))
 (segment (start 155 87) (end 155 73) (width 1.5) (layer "F.Cu") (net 4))
 (segment (start 151 91) (end 155 87) (width 1.5) (layer "F.Cu") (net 4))
 (segment (start 146.7 95.83) (end 156.17 95.83) (width 1.5) (layer "F.Cu") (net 1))
 (segment (start 156.17 95.83) (end 165 87) (width 1.5) (layer "F.Cu") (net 1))
 (segment (start 165 87) (end 165 73) (width 1.5) (layer "F.Cu") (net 1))
 (segment (start 96 101) (end 97 100) (width 1.5) (layer "F.Cu") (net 11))
 (segment (start 63 101) (end 96 101) (width 1.5) (layer "F.Cu") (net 11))
 (segment (start 97 100) (end 97 95.83) (width 1.5) (layer "F.Cu") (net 11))
 (segment (start 61 99) (end 63 101) (width 1.5) (layer "F.Cu") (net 11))
 (segment (start 61 95.83) (end 61 99) (width 1.5) (layer "F.Cu") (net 11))
 (segment (start 63.15 92.15) (end 62 91) (width 1.5) (layer "B.Cu") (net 14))
 (segment (start 94.85 93.15) (end 94.85 98.15) (width 1.5) (layer "B.Cu") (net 14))
 (segment (start 64 100) (end 63.15 99.15) (width 1.5) (layer "B.Cu") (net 14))
 (segment (start 62 91) (end 61 91) (width 1.5) (layer "B.Cu") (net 14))
 (segment (start 94.85 98.15) (end 93 100) (width 1.5) (layer "B.Cu") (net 14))
 (segment (start 97 91) (end 94.85 93.15) (width 1.5) (layer "B.Cu") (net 14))
 (segment (start 63.15 99.15) (end 63.15 92.15) (width 1.5) (layer "B.Cu") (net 14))
 (segment (start 93 100) (end 64 100) (width 1.5) (layer "B.Cu") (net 14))
 (segment (start 61.17 86.17) (end 61 86.17) (width 1.5) (layer "F.Cu") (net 17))
 (segment (start 97 86.17) (end 94.45 88.72) (width 1.5) (layer "F.Cu") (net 17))
 (segment (start 63.15 98.15) (end 63.15 88.15) (width 1.5) (layer "F.Cu") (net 17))
 (segment (start 64 99) (end 63.15 98.15) (width 1.5) (layer "F.Cu") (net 17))
 (segment (start 94.45 88.72) (end 94.45 98.45) (width 1.5) (layer "F.Cu") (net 17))
 (segment (start 93.9 99) (end 64 99) (width 1.5) (layer "F.Cu") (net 17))
 (segment (start 63.15 88.15) (end 61.17 86.17) (width 1.5) (layer "F.Cu") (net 17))
 (segment (start 94.45 98.45) (end 93.9 99) (width 1.5) (layer "F.Cu") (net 17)))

